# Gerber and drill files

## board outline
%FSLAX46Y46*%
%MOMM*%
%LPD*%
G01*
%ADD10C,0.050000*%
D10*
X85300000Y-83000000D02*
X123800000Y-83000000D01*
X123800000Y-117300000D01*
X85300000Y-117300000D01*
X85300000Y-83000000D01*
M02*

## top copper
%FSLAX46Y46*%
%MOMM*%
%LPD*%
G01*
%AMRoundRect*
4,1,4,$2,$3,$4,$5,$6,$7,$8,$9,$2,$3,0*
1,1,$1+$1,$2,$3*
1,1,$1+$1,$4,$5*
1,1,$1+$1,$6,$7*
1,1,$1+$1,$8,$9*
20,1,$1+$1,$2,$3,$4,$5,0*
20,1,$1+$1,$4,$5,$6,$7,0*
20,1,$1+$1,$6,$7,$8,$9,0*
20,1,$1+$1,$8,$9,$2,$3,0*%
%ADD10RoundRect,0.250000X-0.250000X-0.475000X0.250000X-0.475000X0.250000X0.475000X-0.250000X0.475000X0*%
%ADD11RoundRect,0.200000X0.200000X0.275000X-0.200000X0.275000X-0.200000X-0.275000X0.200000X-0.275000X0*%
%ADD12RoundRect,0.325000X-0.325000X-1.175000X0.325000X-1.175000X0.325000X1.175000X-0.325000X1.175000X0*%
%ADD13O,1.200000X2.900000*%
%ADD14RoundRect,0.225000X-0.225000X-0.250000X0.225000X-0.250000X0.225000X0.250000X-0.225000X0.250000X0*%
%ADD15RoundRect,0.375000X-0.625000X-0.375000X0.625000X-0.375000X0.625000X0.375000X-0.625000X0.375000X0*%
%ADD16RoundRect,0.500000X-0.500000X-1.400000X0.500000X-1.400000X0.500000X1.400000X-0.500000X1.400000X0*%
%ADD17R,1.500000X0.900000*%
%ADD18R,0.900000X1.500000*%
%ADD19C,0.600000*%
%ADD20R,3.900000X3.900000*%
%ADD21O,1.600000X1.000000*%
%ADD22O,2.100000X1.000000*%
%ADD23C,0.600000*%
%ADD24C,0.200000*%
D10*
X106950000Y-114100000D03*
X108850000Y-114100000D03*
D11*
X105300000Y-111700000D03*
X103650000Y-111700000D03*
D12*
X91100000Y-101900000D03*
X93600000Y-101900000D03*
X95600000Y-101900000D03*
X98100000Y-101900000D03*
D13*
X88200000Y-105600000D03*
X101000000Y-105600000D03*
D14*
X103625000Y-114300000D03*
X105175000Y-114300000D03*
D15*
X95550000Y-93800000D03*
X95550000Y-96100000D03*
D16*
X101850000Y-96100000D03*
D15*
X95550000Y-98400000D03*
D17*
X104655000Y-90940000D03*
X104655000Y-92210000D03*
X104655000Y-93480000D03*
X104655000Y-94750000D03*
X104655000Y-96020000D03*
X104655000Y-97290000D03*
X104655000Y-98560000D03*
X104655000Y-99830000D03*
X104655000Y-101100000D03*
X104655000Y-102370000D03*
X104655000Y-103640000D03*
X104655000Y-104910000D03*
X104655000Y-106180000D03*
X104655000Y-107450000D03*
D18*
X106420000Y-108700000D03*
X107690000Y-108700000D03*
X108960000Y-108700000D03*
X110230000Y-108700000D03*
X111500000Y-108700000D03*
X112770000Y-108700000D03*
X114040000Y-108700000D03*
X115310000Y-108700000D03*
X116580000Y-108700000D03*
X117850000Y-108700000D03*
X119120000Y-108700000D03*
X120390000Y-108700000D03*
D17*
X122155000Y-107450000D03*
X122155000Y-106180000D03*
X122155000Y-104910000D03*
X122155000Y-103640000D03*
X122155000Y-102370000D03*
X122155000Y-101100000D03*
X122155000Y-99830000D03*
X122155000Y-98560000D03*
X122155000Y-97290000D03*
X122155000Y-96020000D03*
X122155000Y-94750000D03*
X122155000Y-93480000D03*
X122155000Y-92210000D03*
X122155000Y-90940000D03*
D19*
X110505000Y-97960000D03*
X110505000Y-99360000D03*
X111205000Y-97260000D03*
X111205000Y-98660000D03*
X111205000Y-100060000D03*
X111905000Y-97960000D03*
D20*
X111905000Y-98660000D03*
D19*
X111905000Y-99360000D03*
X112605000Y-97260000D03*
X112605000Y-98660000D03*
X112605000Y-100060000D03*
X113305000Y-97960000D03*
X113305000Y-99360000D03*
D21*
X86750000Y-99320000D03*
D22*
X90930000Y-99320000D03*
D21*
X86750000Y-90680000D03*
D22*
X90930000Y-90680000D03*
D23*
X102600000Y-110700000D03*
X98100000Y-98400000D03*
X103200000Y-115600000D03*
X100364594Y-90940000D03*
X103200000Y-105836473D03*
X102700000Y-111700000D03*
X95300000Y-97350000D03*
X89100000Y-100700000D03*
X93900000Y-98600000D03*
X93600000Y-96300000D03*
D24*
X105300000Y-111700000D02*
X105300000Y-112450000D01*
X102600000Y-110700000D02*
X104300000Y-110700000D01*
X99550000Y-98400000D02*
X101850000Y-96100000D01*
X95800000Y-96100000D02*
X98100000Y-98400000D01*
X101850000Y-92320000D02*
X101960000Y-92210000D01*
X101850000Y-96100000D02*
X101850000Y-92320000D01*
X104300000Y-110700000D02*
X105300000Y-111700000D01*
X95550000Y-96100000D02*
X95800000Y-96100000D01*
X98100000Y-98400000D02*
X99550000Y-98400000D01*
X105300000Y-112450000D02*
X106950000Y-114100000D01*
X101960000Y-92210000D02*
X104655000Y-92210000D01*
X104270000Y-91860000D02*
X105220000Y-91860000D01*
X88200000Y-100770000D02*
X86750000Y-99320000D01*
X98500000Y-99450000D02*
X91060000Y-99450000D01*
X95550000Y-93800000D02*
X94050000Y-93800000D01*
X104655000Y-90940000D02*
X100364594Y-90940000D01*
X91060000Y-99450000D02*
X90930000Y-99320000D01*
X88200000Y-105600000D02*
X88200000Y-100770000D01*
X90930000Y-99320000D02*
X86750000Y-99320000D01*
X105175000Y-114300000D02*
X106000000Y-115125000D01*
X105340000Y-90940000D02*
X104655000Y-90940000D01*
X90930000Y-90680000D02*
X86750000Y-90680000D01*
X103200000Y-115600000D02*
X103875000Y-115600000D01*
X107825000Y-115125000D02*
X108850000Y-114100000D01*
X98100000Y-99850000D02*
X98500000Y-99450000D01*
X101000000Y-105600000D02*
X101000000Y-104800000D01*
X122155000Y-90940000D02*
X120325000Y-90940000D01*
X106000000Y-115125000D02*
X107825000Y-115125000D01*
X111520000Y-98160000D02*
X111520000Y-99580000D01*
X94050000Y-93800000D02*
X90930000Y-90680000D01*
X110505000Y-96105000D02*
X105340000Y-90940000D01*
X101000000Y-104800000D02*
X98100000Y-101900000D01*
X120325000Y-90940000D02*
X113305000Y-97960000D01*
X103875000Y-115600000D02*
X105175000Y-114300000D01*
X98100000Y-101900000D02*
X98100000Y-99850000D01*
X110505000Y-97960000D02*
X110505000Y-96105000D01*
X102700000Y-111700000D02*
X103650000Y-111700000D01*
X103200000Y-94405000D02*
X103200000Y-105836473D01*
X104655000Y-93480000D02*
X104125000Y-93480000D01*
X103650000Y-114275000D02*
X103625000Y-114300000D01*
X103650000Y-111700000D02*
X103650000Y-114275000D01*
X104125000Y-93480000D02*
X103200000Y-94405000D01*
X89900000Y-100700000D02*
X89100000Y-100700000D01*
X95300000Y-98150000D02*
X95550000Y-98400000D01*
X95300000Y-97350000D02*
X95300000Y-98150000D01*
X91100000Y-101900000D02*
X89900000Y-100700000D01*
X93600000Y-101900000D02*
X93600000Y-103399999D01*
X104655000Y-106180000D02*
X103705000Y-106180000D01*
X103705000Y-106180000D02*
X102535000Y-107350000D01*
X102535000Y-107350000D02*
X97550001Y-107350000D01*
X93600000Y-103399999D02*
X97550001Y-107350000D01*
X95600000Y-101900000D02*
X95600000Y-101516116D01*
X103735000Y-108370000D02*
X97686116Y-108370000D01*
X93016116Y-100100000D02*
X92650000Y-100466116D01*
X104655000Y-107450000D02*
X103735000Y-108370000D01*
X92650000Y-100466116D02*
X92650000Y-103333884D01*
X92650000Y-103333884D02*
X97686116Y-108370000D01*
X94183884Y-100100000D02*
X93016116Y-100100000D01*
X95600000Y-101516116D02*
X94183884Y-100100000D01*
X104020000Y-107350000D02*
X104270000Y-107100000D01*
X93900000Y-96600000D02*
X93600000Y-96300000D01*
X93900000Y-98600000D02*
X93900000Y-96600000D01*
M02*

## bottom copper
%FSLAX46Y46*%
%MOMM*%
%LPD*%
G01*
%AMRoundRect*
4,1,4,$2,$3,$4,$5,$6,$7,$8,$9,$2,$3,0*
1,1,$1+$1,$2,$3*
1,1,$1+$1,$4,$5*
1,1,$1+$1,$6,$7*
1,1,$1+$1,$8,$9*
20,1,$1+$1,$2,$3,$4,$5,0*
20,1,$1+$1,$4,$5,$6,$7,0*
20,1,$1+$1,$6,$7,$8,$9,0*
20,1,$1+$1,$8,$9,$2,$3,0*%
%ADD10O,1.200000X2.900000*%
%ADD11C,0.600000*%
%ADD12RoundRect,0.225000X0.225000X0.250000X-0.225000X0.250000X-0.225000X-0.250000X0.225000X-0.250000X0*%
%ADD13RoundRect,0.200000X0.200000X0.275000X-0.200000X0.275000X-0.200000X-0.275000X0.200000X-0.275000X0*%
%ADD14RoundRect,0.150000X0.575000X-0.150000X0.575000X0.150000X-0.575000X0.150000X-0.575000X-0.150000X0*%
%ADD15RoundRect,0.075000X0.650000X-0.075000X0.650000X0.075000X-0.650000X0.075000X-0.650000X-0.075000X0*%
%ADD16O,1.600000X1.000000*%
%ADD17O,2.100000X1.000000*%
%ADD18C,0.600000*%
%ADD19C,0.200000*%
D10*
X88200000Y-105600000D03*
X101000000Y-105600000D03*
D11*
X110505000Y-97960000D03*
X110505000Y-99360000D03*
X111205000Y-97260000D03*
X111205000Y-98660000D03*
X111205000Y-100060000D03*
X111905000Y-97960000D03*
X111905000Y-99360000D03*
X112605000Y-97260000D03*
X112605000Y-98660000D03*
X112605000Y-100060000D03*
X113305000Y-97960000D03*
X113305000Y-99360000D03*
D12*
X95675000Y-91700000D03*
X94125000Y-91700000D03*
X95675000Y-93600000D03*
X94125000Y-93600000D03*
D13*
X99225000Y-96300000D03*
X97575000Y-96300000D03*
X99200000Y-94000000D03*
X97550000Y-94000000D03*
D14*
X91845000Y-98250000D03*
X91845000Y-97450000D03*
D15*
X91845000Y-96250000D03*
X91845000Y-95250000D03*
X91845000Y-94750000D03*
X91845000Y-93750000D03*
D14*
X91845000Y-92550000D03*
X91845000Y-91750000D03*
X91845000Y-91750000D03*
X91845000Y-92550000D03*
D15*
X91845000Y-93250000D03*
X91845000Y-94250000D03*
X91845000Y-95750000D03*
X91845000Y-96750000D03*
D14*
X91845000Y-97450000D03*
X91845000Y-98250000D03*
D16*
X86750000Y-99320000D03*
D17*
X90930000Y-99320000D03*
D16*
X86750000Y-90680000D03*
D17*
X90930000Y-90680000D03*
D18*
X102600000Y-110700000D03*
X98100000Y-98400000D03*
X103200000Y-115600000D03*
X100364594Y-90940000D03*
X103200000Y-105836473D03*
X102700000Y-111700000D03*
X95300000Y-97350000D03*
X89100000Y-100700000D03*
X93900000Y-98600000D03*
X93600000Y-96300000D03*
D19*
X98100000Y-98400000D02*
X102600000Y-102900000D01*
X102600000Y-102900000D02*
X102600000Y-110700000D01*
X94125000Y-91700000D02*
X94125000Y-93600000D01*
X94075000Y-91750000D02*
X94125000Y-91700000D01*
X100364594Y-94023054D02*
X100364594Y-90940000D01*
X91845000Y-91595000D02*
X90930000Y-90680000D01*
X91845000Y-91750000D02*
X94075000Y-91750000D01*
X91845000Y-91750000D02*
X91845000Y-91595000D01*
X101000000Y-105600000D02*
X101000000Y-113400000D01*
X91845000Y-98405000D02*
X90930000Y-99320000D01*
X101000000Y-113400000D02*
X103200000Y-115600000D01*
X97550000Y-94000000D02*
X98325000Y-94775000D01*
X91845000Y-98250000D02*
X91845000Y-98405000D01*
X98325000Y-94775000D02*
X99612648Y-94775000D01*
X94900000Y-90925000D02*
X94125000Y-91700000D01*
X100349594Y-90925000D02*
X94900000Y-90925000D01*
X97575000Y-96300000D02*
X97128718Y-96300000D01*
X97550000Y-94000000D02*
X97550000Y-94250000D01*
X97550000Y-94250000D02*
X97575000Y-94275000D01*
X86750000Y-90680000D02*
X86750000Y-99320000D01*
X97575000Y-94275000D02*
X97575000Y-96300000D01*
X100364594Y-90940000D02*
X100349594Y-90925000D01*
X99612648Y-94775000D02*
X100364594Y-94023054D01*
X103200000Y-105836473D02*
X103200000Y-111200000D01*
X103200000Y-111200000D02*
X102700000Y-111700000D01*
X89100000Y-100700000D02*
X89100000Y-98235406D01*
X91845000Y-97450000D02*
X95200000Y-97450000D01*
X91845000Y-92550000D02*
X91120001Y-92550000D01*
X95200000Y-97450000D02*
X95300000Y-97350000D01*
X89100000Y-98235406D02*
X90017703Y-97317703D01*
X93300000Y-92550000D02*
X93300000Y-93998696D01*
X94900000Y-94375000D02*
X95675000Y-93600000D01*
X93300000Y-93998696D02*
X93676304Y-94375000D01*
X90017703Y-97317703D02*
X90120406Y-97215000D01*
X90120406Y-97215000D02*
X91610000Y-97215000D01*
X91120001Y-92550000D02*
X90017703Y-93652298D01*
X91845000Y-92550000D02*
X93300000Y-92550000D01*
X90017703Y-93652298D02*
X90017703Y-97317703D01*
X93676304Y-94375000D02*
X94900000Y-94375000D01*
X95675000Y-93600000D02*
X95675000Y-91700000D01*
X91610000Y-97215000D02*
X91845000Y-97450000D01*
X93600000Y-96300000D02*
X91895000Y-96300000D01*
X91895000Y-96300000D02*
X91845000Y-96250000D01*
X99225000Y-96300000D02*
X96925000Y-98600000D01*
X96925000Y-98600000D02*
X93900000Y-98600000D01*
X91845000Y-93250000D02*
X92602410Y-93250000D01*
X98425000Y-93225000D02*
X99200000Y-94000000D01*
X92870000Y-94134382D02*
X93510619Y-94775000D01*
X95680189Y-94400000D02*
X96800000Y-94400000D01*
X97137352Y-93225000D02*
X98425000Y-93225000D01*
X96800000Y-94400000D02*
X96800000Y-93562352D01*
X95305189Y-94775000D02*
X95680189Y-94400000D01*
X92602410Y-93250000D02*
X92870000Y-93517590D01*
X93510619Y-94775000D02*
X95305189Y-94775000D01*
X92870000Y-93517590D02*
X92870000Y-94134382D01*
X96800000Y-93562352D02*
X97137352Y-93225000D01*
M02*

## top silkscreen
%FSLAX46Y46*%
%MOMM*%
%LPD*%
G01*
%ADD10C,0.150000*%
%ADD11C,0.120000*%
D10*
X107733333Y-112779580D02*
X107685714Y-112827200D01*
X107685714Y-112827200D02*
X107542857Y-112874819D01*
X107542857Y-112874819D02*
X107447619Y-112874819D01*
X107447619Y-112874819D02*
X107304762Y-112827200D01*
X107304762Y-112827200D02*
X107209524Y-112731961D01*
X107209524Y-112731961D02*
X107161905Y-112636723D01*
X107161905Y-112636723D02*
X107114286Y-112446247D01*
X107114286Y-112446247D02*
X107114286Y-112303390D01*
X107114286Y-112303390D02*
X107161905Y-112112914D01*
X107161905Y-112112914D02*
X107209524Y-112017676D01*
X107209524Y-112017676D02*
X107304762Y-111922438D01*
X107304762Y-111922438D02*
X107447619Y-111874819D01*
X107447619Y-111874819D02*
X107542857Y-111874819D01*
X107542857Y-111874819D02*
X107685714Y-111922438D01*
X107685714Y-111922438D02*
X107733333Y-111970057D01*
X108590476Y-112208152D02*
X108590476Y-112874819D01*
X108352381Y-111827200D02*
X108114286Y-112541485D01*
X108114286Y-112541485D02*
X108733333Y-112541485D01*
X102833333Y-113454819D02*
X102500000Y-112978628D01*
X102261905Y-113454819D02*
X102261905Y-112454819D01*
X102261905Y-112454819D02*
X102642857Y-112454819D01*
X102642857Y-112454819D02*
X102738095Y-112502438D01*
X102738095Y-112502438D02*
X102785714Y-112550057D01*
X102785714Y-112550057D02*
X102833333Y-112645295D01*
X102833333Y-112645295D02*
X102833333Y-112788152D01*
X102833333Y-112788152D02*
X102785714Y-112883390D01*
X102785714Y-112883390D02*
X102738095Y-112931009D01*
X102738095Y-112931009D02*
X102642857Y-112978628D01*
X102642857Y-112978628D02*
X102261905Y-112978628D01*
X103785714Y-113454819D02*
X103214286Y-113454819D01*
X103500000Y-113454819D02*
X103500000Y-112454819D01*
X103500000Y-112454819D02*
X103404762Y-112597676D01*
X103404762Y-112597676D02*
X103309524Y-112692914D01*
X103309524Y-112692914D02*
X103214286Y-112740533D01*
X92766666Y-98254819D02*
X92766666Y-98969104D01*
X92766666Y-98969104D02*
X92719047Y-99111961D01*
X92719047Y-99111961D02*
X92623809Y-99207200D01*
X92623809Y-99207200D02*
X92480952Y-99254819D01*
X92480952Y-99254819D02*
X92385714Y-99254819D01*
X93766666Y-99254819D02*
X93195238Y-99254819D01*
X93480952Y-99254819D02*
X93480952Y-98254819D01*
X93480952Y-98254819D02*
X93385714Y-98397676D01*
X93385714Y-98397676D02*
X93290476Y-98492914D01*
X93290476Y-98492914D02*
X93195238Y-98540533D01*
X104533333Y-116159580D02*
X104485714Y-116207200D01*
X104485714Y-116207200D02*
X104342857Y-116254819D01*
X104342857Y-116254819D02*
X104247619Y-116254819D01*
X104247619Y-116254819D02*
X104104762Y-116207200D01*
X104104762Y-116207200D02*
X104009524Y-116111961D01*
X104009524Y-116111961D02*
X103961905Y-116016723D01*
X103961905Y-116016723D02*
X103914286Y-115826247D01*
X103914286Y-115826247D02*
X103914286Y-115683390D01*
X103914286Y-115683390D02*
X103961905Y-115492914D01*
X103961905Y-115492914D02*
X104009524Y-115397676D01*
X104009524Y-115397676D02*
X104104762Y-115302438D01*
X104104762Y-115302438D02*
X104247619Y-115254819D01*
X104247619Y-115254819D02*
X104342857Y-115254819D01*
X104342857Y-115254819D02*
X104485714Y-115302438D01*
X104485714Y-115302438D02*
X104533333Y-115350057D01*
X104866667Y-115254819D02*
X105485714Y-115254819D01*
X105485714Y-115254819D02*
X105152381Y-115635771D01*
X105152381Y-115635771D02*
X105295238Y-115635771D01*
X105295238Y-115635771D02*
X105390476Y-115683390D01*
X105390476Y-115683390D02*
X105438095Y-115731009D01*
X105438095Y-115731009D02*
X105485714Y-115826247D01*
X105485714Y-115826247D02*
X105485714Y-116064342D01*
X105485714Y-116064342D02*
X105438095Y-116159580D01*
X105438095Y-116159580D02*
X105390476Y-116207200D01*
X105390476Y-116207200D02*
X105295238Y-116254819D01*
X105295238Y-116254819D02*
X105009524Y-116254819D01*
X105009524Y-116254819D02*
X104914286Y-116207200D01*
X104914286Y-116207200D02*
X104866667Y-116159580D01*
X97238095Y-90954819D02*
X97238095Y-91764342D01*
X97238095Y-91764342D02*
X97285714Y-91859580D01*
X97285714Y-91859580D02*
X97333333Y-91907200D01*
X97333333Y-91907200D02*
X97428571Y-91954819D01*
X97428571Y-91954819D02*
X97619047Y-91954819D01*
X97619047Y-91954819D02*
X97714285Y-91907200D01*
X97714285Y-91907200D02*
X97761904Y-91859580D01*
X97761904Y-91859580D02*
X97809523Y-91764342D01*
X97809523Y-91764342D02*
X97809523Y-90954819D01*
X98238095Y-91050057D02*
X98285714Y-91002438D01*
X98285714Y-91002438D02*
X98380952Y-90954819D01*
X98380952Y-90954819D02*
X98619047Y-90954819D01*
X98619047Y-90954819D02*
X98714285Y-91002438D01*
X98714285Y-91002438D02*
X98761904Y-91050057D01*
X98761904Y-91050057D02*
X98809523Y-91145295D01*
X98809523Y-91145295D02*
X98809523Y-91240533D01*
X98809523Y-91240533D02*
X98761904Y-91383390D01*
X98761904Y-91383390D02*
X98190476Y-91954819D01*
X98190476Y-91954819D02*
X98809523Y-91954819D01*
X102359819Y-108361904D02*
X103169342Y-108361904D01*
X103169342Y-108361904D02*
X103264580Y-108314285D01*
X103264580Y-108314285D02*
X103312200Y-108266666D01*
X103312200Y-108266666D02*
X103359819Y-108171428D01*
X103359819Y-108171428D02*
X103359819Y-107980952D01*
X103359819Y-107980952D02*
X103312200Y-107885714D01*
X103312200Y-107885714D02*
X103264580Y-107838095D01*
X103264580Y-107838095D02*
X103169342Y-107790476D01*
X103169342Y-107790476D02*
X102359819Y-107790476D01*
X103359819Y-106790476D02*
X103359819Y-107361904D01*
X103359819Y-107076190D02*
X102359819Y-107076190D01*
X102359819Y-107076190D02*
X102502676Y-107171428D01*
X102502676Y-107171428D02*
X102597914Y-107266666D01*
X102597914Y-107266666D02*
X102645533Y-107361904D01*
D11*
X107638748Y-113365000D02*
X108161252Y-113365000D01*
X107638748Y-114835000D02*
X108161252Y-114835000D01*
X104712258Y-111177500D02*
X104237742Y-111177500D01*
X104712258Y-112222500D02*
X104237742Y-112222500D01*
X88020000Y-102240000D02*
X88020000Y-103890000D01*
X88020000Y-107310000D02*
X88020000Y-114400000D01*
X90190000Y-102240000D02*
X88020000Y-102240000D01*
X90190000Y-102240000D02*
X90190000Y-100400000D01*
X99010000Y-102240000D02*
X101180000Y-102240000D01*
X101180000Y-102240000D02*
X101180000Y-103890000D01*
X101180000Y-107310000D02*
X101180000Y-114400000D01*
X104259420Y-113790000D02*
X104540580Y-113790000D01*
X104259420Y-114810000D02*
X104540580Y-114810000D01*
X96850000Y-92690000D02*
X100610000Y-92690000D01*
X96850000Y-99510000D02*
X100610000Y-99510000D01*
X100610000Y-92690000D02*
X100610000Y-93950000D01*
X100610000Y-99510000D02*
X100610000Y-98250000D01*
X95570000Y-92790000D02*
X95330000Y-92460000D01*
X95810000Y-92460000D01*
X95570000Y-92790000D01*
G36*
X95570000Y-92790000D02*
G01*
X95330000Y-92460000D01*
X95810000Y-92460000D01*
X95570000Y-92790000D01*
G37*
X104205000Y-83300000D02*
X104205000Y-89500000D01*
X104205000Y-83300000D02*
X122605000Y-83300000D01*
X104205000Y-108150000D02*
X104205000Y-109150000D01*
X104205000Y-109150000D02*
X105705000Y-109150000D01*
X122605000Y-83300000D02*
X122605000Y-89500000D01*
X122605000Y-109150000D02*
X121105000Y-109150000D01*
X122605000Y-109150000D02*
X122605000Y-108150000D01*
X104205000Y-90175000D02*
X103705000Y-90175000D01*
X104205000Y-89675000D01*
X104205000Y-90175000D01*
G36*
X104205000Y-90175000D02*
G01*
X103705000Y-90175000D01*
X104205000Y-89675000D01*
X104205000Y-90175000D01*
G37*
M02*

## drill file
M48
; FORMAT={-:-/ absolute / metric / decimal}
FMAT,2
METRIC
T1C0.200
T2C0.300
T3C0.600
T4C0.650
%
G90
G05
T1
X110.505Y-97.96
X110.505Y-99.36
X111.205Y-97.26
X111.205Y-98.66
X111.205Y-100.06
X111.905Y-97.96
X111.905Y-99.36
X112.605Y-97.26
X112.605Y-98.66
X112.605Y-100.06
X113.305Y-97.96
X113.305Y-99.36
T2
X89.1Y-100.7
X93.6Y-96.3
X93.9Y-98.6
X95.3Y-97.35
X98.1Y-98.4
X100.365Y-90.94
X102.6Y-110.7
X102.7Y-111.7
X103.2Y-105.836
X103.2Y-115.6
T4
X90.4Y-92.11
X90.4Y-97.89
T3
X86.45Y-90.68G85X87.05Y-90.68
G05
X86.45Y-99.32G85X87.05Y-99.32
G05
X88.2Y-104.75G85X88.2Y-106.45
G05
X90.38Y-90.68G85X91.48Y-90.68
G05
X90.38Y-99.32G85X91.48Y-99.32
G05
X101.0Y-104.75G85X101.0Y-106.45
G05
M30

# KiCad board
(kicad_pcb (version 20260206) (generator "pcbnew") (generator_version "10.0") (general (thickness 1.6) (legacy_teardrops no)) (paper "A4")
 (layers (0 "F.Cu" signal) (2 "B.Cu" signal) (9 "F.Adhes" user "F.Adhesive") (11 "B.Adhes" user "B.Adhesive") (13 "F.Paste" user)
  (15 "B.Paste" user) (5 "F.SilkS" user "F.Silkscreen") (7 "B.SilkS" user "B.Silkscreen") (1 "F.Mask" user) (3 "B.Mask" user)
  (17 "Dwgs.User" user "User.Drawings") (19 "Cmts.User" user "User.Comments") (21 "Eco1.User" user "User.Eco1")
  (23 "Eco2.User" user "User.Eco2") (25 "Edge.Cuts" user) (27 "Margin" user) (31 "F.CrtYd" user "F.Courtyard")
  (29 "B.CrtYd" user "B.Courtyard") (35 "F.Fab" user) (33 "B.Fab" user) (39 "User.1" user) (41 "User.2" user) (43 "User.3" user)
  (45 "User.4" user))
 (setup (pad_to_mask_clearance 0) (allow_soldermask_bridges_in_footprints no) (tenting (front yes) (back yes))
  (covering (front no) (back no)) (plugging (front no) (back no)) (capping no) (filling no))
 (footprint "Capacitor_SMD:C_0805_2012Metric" (layer "F.Cu") (at 107.9 114.1)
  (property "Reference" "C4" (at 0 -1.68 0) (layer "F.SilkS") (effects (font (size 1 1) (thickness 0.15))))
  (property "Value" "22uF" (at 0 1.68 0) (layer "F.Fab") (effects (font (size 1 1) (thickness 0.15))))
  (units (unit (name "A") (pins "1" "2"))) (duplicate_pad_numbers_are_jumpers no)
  (fp_line (start -0.261252 -0.735) (end 0.261252 -0.735) (stroke (width 0.12) (type solid)) (layer "F.SilkS"))
  (fp_line (start -0.261252 0.735) (end 0.261252 0.735) (stroke (width 0.12) (type solid)) (layer "F.SilkS"))
  (pad "1" smd roundrect (at -0.95 0) (size 1 1.45) (layers "F.Cu" "F.Mask" "F.Paste") (roundrect_rratio 0.25) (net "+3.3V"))
  (pad "2" smd roundrect (at 0.95 0) (size 1 1.45) (layers "F.Cu" "F.Mask" "F.Paste") (roundrect_rratio 0.25) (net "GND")))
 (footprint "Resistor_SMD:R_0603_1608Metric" (layer "F.Cu") (at 104.475 111.7 180)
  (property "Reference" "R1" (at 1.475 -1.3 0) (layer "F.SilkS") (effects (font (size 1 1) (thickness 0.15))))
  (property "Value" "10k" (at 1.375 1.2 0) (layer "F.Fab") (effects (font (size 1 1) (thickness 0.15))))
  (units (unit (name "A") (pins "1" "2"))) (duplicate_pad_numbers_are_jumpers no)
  (fp_line (start -0.237258 0.5225) (end 0.237258 0.5225) (stroke (width 0.12) (type solid)) (layer "F.SilkS"))
  (fp_line (start -0.237258 -0.5225) (end 0.237258 -0.5225) (stroke (width 0.12) (type solid)) (layer "F.SilkS"))
  (pad "1" smd roundrect (at -0.825 0 180) (size 0.8 0.95) (layers "F.Cu" "F.Mask" "F.Paste") (roundrect_rratio 0.25) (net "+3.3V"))
  (pad "2" smd roundrect (at 0.825 0 180) (size 0.8 0.95) (layers "F.Cu" "F.Mask" "F.Paste") (roundrect_rratio 0.25) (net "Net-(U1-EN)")))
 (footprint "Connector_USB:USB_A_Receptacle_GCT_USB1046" (layer "F.Cu") (at 94.6 109.15)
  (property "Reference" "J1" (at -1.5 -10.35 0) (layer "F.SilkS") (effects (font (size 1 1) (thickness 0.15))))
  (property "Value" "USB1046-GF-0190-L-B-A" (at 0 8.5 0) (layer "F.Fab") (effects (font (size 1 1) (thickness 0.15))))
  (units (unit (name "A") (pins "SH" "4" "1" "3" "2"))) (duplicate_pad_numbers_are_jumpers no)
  (fp_line (start -6.58 -6.91) (end -6.58 -5.26) (stroke (width 0.12) (type default)) (layer "F.SilkS"))
  (fp_line (start -6.58 -1.84) (end -6.58 5.25) (stroke (width 0.12) (type default)) (layer "F.SilkS"))
  (fp_line (start -4.41 -6.91) (end -6.58 -6.91) (stroke (width 0.12) (type default)) (layer "F.SilkS"))
  (fp_line (start -4.41 -6.91) (end -4.41 -8.75) (stroke (width 0.12) (type default)) (layer "F.SilkS"))
  (fp_line (start 4.41 -6.91) (end 6.58 -6.91) (stroke (width 0.12) (type default)) (layer "F.SilkS"))
  (fp_line (start 6.58 -6.91) (end 6.58 -5.26) (stroke (width 0.12) (type default)) (layer "F.SilkS"))
  (fp_line (start 6.58 -1.84) (end 6.58 5.25) (stroke (width 0.12) (type default)) (layer "F.SilkS"))
  (pad "" smd oval (at -6.4 -3.55) (size 1.2 2.9) (layers "F.Paste") (thermal_bridge_angle 45))
  (pad "" smd oval (at 6.4 -3.55) (size 1.2 2.9) (layers "F.Paste") (thermal_bridge_angle 45))
  (pad "1" smd roundrect (at -3.5 -7.25) (size 1.3 3) (layers "F.Cu" "F.Mask" "F.Paste") (roundrect_rratio 0.25) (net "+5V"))
  (pad "2" smd roundrect (at -1 -7.25) (size 1.3 3) (layers "F.Cu" "F.Mask" "F.Paste") (roundrect_rratio 0.25) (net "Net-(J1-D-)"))
  (pad "3" smd roundrect (at 1 -7.25) (size 1.3 3) (layers "F.Cu" "F.Mask" "F.Paste") (roundrect_rratio 0.25) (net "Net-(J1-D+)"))
  (pad "4" smd roundrect (at 3.5 -7.25) (size 1.3 3) (layers "F.Cu" "F.Mask" "F.Paste") (roundrect_rratio 0.25) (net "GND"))
  (pad "SH" thru_hole oval (at -6.4 -3.55) (size 1.2 2.9) (drill oval 0.6 2.3) (layers "*.Cu" "*.Mask") (remove_unused_layers no)
   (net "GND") (thermal_bridge_angle 45))
  (pad "SH" thru_hole oval (at 6.4 -3.55) (size 1.2 2.9) (drill oval 0.6 2.3) (layers "*.Cu" "*.Mask") (remove_unused_layers no) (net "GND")
   (thermal_bridge_angle 45)))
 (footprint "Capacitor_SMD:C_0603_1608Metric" (layer "F.Cu") (at 104.4 114.3)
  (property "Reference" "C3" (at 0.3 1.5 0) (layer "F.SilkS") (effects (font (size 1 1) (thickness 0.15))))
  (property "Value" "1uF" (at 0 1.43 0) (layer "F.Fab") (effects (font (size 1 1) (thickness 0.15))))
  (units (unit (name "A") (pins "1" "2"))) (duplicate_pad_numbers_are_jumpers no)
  (fp_line (start -0.14058 -0.51) (end 0.14058 -0.51) (stroke (width 0.12) (type solid)) (layer "F.SilkS"))
  (fp_line (start -0.14058 0.51) (end 0.14058 0.51) (stroke (width 0.12) (type solid)) (layer "F.SilkS"))
  (pad "1" smd roundrect (at -0.775 0) (size 0.9 0.95) (layers "F.Cu" "F.Mask" "F.Paste") (roundrect_rratio 0.25) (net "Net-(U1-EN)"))
  (pad "2" smd roundrect (at 0.775 0) (size 0.9 0.95) (layers "F.Cu" "F.Mask" "F.Paste") (roundrect_rratio 0.25) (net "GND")))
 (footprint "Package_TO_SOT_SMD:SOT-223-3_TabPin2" (layer "F.Cu") (at 98.7 96.1)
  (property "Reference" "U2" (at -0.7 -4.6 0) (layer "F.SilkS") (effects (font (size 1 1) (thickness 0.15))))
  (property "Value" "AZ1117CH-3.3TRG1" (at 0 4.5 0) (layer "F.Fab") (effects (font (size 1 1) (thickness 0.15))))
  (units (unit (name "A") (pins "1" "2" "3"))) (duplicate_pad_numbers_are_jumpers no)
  (fp_line (start -1.85 -3.41) (end 1.91 -3.41) (stroke (width 0.12) (type solid)) (layer "F.SilkS"))
  (fp_line (start -1.85 3.41) (end 1.91 3.41) (stroke (width 0.12) (type solid)) (layer "F.SilkS"))
  (fp_line (start 1.91 -3.41) (end 1.91 -2.15) (stroke (width 0.12) (type solid)) (layer "F.SilkS"))
  (fp_line (start 1.91 3.41) (end 1.91 2.15) (stroke (width 0.12) (type solid)) (layer "F.SilkS"))
  (fp_poly
   (pts (xy -3.13 -3.31) (xy -3.37 -3.64) (xy -2.89 -3.64) (xy -3.13 -3.31)) (stroke (width 0.12) (type solid)) (fill yes) (layer "F.SilkS"))
  (pad "1" smd roundrect (at -3.15 -2.3) (size 2 1.5) (layers "F.Cu" "F.Mask" "F.Paste") (roundrect_rratio 0.25) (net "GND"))
  (pad "2" smd roundrect (at -3.15 0) (size 2 1.5) (layers "F.Cu" "F.Mask" "F.Paste") (roundrect_rratio 0.25) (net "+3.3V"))
  (pad "2" smd roundrect (at 3.15 0) (size 2 3.8) (layers "F.Cu" "F.Mask" "F.Paste") (roundrect_rratio 0.25) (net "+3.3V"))
  (pad "3" smd roundrect (at -3.15 2.3) (size 2 1.5) (layers "F.Cu" "F.Mask" "F.Paste") (roundrect_rratio 0.25) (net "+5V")))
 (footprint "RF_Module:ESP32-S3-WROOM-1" (layer "F.Cu") (at 113.405 96.2)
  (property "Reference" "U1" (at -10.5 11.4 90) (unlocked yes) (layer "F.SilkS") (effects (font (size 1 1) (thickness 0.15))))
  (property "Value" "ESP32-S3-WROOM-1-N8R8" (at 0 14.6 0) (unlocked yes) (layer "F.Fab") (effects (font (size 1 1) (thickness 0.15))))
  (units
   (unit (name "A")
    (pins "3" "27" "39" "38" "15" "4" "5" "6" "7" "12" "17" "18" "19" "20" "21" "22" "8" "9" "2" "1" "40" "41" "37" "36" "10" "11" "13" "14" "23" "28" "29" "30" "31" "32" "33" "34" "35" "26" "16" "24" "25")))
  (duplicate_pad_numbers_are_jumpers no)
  (fp_line (start -9.2 -12.9) (end -9.2 -6.7) (stroke (width 0.12) (type solid)) (layer "F.SilkS"))
  (fp_line (start -9.2 -12.9) (end 9.2 -12.9) (stroke (width 0.12) (type solid)) (layer "F.SilkS"))
  (fp_line (start -9.2 11.95) (end -9.2 12.95) (stroke (width 0.12) (type solid)) (layer "F.SilkS"))
  (fp_line (start -9.2 12.95) (end -7.7 12.95) (stroke (width 0.12) (type solid)) (layer "F.SilkS"))
  (fp_line (start 9.2 -12.9) (end 9.2 -6.7) (stroke (width 0.12) (type solid)) (layer "F.SilkS"))
  (fp_line (start 9.2 12.95) (end 7.7 12.95) (stroke (width 0.12) (type solid)) (layer "F.SilkS"))
  (fp_line (start 9.2 12.95) (end 9.2 11.95) (stroke (width 0.12) (type solid)) (layer "F.SilkS"))
  (fp_poly
   (pts (xy -9.2 -6.025) (xy -9.7 -6.025) (xy -9.2 -6.525) (xy -9.2 -6.025)) (stroke (width 0.12) (type solid)) (fill yes) (layer "F.SilkS"))
  (pad "" smd rect (at -2.9 1.06) (size 0.9 0.9) (layers "F.Paste"))
  (pad "" smd rect (at -2.9 2.46 270) (size 0.9 0.9) (layers "F.Paste"))
  (pad "" smd rect (at -2.9 3.86) (size 0.9 0.9) (layers "F.Paste"))
  (pad "" smd rect (at -1.5 1.06 270) (size 0.9 0.9) (layers "F.Paste"))
  (pad "" smd rect (at -1.5 2.46 270) (size 0.9 0.9) (layers "F.Paste"))
  (pad "" smd rect (at -1.5 3.86 270) (size 0.9 0.9) (layers "F.Paste"))
  (pad "" smd rect (at -0.1 1.06 270) (size 0.9 0.9) (layers "F.Paste"))
  (pad "" smd rect (at -0.1 2.46 270) (size 0.9 0.9) (layers "F.Paste"))
  (pad "" smd rect (at -0.1 3.86 270) (size 0.9 0.9) (layers "F.Paste"))
  (pad "1" smd rect (at -8.75 -5.26) (size 1.5 0.9) (layers "F.Cu" "F.Mask" "F.Paste") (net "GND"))
  (pad "2" smd rect (at -8.75 -3.99) (size 1.5 0.9) (layers "F.Cu" "F.Mask" "F.Paste") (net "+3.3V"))
  (pad "3" smd rect (at -8.75 -2.72) (size 1.5 0.9) (layers "F.Cu" "F.Mask" "F.Paste") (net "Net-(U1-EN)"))
  (pad "4" smd rect (at -8.75 -1.45) (size 1.5 0.9) (layers "F.Cu" "F.Mask" "F.Paste") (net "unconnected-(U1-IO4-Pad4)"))
  (pad "5" smd rect (at -8.75 -0.18) (size 1.5 0.9) (layers "F.Cu" "F.Mask" "F.Paste") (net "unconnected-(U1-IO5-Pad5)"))
  (pad "6" smd rect (at -8.75 1.09) (size 1.5 0.9) (layers "F.Cu" "F.Mask" "F.Paste") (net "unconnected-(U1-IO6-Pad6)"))
  (pad "7" smd rect (at -8.75 2.36) (size 1.5 0.9) (layers "F.Cu" "F.Mask" "F.Paste") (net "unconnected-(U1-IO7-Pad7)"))
  (pad "8" smd rect (at -8.75 3.63) (size 1.5 0.9) (layers "F.Cu" "F.Mask" "F.Paste") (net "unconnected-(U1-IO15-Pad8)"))
  (pad "9" smd rect (at -8.75 4.9) (size 1.5 0.9) (layers "F.Cu" "F.Mask" "F.Paste") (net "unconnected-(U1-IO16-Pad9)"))
  (pad "10" smd rect (at -8.75 6.17) (size 1.5 0.9) (layers "F.Cu" "F.Mask" "F.Paste") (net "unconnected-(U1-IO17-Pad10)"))
  (pad "11" smd rect (at -8.75 7.44) (size 1.5 0.9) (layers "F.Cu" "F.Mask" "F.Paste") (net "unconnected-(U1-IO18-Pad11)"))
  (pad "12" smd rect (at -8.75 8.71) (size 1.5 0.9) (layers "F.Cu" "F.Mask" "F.Paste") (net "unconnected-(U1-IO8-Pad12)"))
  (pad "13" smd rect (at -8.75 9.98) (size 1.5 0.9) (layers "F.Cu" "F.Mask" "F.Paste") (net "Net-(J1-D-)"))
  (pad "14" smd rect (at -8.75 11.25 180) (size 1.5 0.9) (layers "F.Cu" "F.Mask" "F.Paste") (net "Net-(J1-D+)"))
  (pad "15" smd rect (at -6.985 12.5 270) (size 1.5 0.9) (layers "F.Cu" "F.Mask" "F.Paste") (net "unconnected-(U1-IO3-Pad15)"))
  (pad "16" smd rect (at -5.715 12.5 270) (size 1.5 0.9) (layers "F.Cu" "F.Mask" "F.Paste") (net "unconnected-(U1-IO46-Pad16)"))
  (pad "17" smd rect (at -4.445 12.5 270) (size 1.5 0.9) (layers "F.Cu" "F.Mask" "F.Paste") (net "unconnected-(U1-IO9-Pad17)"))
  (pad "18" smd rect (at -3.175 12.5 270) (size 1.5 0.9) (layers "F.Cu" "F.Mask" "F.Paste") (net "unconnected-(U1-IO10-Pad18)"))
  (pad "19" smd rect (at -1.905 12.5 270) (size 1.5 0.9) (layers "F.Cu" "F.Mask" "F.Paste") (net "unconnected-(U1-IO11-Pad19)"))
  (pad "20" smd rect (at -0.635 12.5 270) (size 1.5 0.9) (layers "F.Cu" "F.Mask" "F.Paste") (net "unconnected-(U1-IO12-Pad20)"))
  (pad "21" smd rect (at 0.635 12.5 270) (size 1.5 0.9) (layers "F.Cu" "F.Mask" "F.Paste") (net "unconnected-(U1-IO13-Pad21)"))
  (pad "22" smd rect (at 1.905 12.5 270) (size 1.5 0.9) (layers "F.Cu" "F.Mask" "F.Paste") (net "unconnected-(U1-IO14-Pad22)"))
  (pad "23" smd rect (at 3.175 12.5 270) (size 1.5 0.9) (layers "F.Cu" "F.Mask" "F.Paste") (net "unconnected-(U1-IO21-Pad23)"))
  (pad "24" smd rect (at 4.445 12.5 270) (size 1.5 0.9) (layers "F.Cu" "F.Mask" "F.Paste") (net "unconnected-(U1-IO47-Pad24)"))
  (pad "25" smd rect (at 5.715 12.5 270) (size 1.5 0.9) (layers "F.Cu" "F.Mask" "F.Paste") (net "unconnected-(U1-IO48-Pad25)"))
  (pad "26" smd rect (at 6.985 12.5 270) (size 1.5 0.9) (layers "F.Cu" "F.Mask" "F.Paste") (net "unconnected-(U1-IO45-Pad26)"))
  (pad "27" smd rect (at 8.75 11.25) (size 1.5 0.9) (layers "F.Cu" "F.Mask" "F.Paste") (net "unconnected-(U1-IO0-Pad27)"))
  (pad "28" smd rect (at 8.75 9.98) (size 1.5 0.9) (layers "F.Cu" "F.Mask" "F.Paste") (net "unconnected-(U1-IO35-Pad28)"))
  (pad "29" smd rect (at 8.75 8.71) (size 1.5 0.9) (layers "F.Cu" "F.Mask" "F.Paste") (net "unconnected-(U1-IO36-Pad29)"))
  (pad "30" smd rect (at 8.75 7.44) (size 1.5 0.9) (layers "F.Cu" "F.Mask" "F.Paste") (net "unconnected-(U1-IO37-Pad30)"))
  (pad "31" smd rect (at 8.75 6.17) (size 1.5 0.9) (layers "F.Cu" "F.Mask" "F.Paste") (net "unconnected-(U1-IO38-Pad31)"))
  (pad "32" smd rect (at 8.75 4.9) (size 1.5 0.9) (layers "F.Cu" "F.Mask" "F.Paste") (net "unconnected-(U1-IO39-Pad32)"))
  (pad "33" smd rect (at 8.75 3.63) (size 1.5 0.9) (layers "F.Cu" "F.Mask" "F.Paste") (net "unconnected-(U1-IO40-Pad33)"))
  (pad "34" smd rect (at 8.75 2.36) (size 1.5 0.9) (layers "F.Cu" "F.Mask" "F.Paste") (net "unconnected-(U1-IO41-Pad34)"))
  (pad "35" smd rect (at 8.75 1.09) (size 1.5 0.9) (layers "F.Cu" "F.Mask" "F.Paste") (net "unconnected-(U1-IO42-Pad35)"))
  (pad "36" smd rect (at 8.75 -0.18) (size 1.5 0.9) (layers "F.Cu" "F.Mask" "F.Paste") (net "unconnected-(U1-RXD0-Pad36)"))
  (pad "37" smd rect (at 8.75 -1.45) (size 1.5 0.9) (layers "F.Cu" "F.Mask" "F.Paste") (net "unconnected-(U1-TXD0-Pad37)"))
  (pad "38" smd rect (at 8.75 -2.72) (size 1.5 0.9) (layers "F.Cu" "F.Mask" "F.Paste") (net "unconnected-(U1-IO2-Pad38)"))
  (pad "39" smd rect (at 8.75 -3.99) (size 1.5 0.9) (layers "F.Cu" "F.Mask" "F.Paste") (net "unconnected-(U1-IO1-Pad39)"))
  (pad "40" smd rect (at 8.75 -5.26) (size 1.5 0.9) (layers "F.Cu" "F.Mask" "F.Paste") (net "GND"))
  (pad "41" thru_hole circle (at -2.9 1.76 90) (size 0.6 0.6) (drill 0.2) (layers "*.Cu" "F.Mask") (remove_unused_layers no) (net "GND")
   (zone_connect 2))
  (pad "41" thru_hole circle (at -2.9 3.16) (size 0.6 0.6) (drill 0.2) (layers "*.Cu" "F.Mask") (remove_unused_layers no) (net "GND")
   (zone_connect 2))
  (pad "41" thru_hole circle (at -2.2 1.06) (size 0.6 0.6) (drill 0.2) (layers "*.Cu" "F.Mask") (remove_unused_layers no) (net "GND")
   (zone_connect 2))
  (pad "41" thru_hole circle (at -2.2 2.46) (size 0.6 0.6) (drill 0.2) (layers "*.Cu" "F.Mask") (remove_unused_layers no) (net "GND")
   (zone_connect 2))
  (pad "41" thru_hole circle (at -2.2 3.86) (size 0.6 0.6) (drill 0.2) (layers "*.Cu" "F.Mask") (remove_unused_layers no) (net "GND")
   (zone_connect 2))
  (pad "41" thru_hole circle (at -1.5 1.76) (size 0.6 0.6) (drill 0.2) (layers "*.Cu" "F.Mask") (remove_unused_layers no) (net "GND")
   (zone_connect 2))
  (pad "41" smd rect (at -1.5 2.46 270) (size 3.9 3.9) (layers "F.Cu" "F.Mask") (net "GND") (zone_connect 2))
  (pad "41" thru_hole circle (at -1.5 3.16) (size 0.6 0.6) (drill 0.2) (layers "*.Cu" "F.Mask") (remove_unused_layers no) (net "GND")
   (zone_connect 2))
  (pad "41" thru_hole circle (at -0.8 1.06) (size 0.6 0.6) (drill 0.2) (layers "*.Cu" "F.Mask") (remove_unused_layers no) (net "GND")
   (zone_connect 2))
  (pad "41" thru_hole circle (at -0.8 2.46) (size 0.6 0.6) (drill 0.2) (layers "*.Cu" "F.Mask") (remove_unused_layers no) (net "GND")
   (zone_connect 2))
  (pad "41" thru_hole circle (at -0.8 3.86) (size 0.6 0.6) (drill 0.2) (layers "*.Cu" "F.Mask") (remove_unused_layers no) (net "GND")
   (zone_connect 2))
  (pad "41" thru_hole circle (at -0.1 1.76) (size 0.6 0.6) (drill 0.2) (layers "*.Cu" "F.Mask") (remove_unused_layers no) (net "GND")
   (zone_connect 2))
  (pad "41" thru_hole circle (at -0.1 3.16) (size 0.6 0.6) (drill 0.2) (layers "*.Cu" "F.Mask") (remove_unused_layers no) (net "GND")
   (zone_connect 2))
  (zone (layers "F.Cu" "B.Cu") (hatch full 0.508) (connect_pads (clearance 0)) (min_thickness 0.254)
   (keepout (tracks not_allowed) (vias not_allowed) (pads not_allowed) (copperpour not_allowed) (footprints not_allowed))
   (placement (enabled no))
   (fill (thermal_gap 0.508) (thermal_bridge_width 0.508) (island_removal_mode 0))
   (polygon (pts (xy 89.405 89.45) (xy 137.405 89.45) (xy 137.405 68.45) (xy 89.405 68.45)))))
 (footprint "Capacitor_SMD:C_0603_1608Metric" (layer "B.Cu") (at 94.9 91.7 180)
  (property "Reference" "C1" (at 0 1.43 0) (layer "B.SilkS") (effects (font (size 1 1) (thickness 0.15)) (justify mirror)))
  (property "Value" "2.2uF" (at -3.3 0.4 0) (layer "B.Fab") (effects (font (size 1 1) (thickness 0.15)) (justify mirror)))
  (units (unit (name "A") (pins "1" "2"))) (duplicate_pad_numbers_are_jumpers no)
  (pad "1" smd roundrect (at -0.775 0 180) (size 0.9 0.95) (layers "B.Cu" "B.Mask" "B.Paste") (roundrect_rratio 0.25) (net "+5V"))
  (pad "2" smd roundrect (at 0.775 0 180) (size 0.9 0.95) (layers "B.Cu" "B.Mask" "B.Paste") (roundrect_rratio 0.25) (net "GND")))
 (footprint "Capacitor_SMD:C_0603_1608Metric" (layer "B.Cu") (at 94.9 93.6 180)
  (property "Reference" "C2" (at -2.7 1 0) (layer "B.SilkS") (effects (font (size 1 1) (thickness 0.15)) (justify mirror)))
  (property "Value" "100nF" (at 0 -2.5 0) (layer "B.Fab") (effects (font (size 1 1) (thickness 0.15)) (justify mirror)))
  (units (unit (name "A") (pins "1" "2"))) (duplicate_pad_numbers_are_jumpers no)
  (pad "1" smd roundrect (at -0.775 0 180) (size 0.9 0.95) (layers "B.Cu" "B.Mask" "B.Paste") (roundrect_rratio 0.25) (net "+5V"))
  (pad "2" smd roundrect (at 0.775 0 180) (size 0.9 0.95) (layers "B.Cu" "B.Mask" "B.Paste") (roundrect_rratio 0.25) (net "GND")))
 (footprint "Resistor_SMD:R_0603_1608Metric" (layer "B.Cu") (at 98.4 96.3 180)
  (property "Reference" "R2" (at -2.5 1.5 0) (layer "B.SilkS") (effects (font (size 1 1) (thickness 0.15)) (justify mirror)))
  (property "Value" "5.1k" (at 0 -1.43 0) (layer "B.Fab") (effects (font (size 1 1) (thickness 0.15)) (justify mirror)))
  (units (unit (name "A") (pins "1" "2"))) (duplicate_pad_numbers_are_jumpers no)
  (pad "1" smd roundrect (at -0.825 0 180) (size 0.8 0.95) (layers "B.Cu" "B.Mask" "B.Paste") (roundrect_rratio 0.25) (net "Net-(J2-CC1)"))
  (pad "2" smd roundrect (at 0.825 0 180) (size 0.8 0.95) (layers "B.Cu" "B.Mask" "B.Paste") (roundrect_rratio 0.25) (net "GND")))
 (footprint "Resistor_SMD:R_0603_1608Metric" (layer "B.Cu") (at 98.375 94 180)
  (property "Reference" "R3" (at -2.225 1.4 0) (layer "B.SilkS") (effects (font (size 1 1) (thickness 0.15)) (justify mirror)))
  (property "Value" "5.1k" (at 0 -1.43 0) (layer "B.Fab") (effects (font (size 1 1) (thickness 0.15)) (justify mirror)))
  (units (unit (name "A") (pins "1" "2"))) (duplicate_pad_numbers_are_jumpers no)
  (pad "1" smd roundrect (at -0.825 0 180) (size 0.8 0.95) (layers "B.Cu" "B.Mask" "B.Paste") (roundrect_rratio 0.25) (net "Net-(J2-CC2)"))
  (pad "2" smd roundrect (at 0.825 0 180) (size 0.8 0.95) (layers "B.Cu" "B.Mask" "B.Paste") (roundrect_rratio 0.25) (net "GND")))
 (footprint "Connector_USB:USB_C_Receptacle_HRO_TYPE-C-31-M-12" (layer "B.Cu") (at 87.8 95 90)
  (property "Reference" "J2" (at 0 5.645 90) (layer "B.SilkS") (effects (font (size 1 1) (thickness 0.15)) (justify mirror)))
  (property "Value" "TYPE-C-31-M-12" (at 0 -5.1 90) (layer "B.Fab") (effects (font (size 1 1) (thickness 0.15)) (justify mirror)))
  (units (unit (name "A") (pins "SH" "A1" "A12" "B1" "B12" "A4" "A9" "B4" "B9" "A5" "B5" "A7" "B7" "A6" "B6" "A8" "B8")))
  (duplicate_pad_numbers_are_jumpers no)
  (pad "" np_thru_hole circle (at -2.89 2.6 90) (size 0.65 0.65) (drill 0.65) (layers "*.Cu" "*.Mask"))
  (pad "" np_thru_hole circle (at 2.89 2.6 90) (size 0.65 0.65) (drill 0.65) (layers "*.Cu" "*.Mask"))
  (pad "A1" smd roundrect (at -3.25 4.045 90) (size 0.6 1.45) (layers "B.Cu" "B.Mask" "B.Paste") (roundrect_rratio 0.25) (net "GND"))
  (pad "A4" smd roundrect (at -2.45 4.045 90) (size 0.6 1.45) (layers "B.Cu" "B.Mask" "B.Paste") (roundrect_rratio 0.25) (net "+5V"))
  (pad "A5" smd roundrect (at -1.25 4.045 90) (size 0.3 1.45) (layers "B.Cu" "B.Mask" "B.Paste") (roundrect_rratio 0.25)
   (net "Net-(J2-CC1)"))
  (pad "A6" smd roundrect (at -0.25 4.045 90) (size 0.3 1.45) (layers "B.Cu" "B.Mask" "B.Paste") (roundrect_rratio 0.25)
   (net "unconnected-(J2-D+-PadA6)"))
  (pad "A7" smd roundrect (at 0.25 4.045 90) (size 0.3 1.45) (layers "B.Cu" "B.Mask" "B.Paste") (roundrect_rratio 0.25)
   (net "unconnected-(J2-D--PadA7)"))
  (pad "A8" smd roundrect (at 1.25 4.045 90) (size 0.3 1.45) (layers "B.Cu" "B.Mask" "B.Paste") (roundrect_rratio 0.25)
   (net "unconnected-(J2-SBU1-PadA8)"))
  (pad "A9" smd roundrect (at 2.45 4.045 90) (size 0.6 1.45) (layers "B.Cu" "B.Mask" "B.Paste") (roundrect_rratio 0.25) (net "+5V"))
  (pad "A12" smd roundrect (at 3.25 4.045 90) (size 0.6 1.45) (layers "B.Cu" "B.Mask" "B.Paste") (roundrect_rratio 0.25) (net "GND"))
  (pad "B1" smd roundrect (at 3.25 4.045 90) (size 0.6 1.45) (layers "B.Cu" "B.Mask" "B.Paste") (roundrect_rratio 0.25) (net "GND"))
  (pad "B4" smd roundrect (at 2.45 4.045 90) (size 0.6 1.45) (layers "B.Cu" "B.Mask" "B.Paste") (roundrect_rratio 0.25) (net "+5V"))
  (pad "B5" smd roundrect (at 1.75 4.045 90) (size 0.3 1.45) (layers "B.Cu" "B.Mask" "B.Paste") (roundrect_rratio 0.25) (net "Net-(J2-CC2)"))
  (pad "B6" smd roundrect (at 0.75 4.045 90) (size 0.3 1.45) (layers "B.Cu" "B.Mask" "B.Paste") (roundrect_rratio 0.25)
   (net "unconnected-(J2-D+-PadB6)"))
  (pad "B7" smd roundrect (at -0.75 4.045 90) (size 0.3 1.45) (layers "B.Cu" "B.Mask" "B.Paste") (roundrect_rratio 0.25)
   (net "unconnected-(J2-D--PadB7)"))
  (pad "B8" smd roundrect (at -1.75 4.045 90) (size 0.3 1.45) (layers "B.Cu" "B.Mask" "B.Paste") (roundrect_rratio 0.25)
   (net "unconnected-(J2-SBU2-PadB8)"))
  (pad "B9" smd roundrect (at -2.45 4.045 90) (size 0.6 1.45) (layers "B.Cu" "B.Mask" "B.Paste") (roundrect_rratio 0.25) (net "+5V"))
  (pad "B12" smd roundrect (at -3.25 4.045 90) (size 0.6 1.45) (layers "B.Cu" "B.Mask" "B.Paste") (roundrect_rratio 0.25) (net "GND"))
  (pad "SH" thru_hole oval (at -4.32 -1.05 90) (size 1 1.6) (drill oval 0.6 1.2) (layers "*.Cu" "*.Mask") (remove_unused_layers no)
   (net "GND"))
  (pad "SH" thru_hole oval (at -4.32 3.13 90) (size 1 2.1) (drill oval 0.6 1.7) (layers "*.Cu" "*.Mask") (remove_unused_layers no)
   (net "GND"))
  (pad "SH" thru_hole oval (at 4.32 -1.05 90) (size 1 1.6) (drill oval 0.6 1.2) (layers "*.Cu" "*.Mask") (remove_unused_layers no)
   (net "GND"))
  (pad "SH" thru_hole oval (at 4.32 3.13 90) (size 1 2.1) (drill oval 0.6 1.7) (layers "*.Cu" "*.Mask") (remove_unused_layers no)
   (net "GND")))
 (gr_rect (start 85.3 83) (end 123.8 117.3) (stroke (width 0.05) (type default)) (fill no) (layer "Edge.Cuts"))
 (segment (start 105.3 111.7) (end 105.3 112.45) (width 0.2) (layer "F.Cu") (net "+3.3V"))
 (segment (start 102.6 110.7) (end 104.3 110.7) (width 0.2) (layer "F.Cu") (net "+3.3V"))
 (segment (start 99.55 98.4) (end 101.85 96.1) (width 0.2) (layer "F.Cu") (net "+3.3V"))
 (segment (start 95.8 96.1) (end 98.1 98.4) (width 0.2) (layer "F.Cu") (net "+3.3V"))
 (segment (start 101.85 92.32) (end 101.96 92.21) (width 0.2) (layer "F.Cu") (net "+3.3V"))
 (segment (start 101.85 96.1) (end 101.85 92.32) (width 0.2) (layer "F.Cu") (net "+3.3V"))
 (segment (start 104.3 110.7) (end 105.3 111.7) (width 0.2) (layer "F.Cu") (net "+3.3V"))
 (segment (start 95.55 96.1) (end 95.8 96.1) (width 0.2) (layer "F.Cu") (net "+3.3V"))
 (segment (start 98.1 98.4) (end 99.55 98.4) (width 0.2) (layer "F.Cu") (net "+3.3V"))
 (segment (start 105.3 112.45) (end 106.95 114.1) (width 0.2) (layer "F.Cu") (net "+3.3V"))
 (segment (start 101.96 92.21) (end 104.655 92.21) (width 0.2) (layer "F.Cu") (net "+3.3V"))
 (segment (start 104.27 91.86) (end 105.22 91.86) (width 0.2) (layer "F.Cu") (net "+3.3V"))
 (via (at 102.6 110.7) (size 0.6) (drill 0.3) (layers "F.Cu" "B.Cu") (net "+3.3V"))
 (via (at 98.1 98.4) (size 0.6) (drill 0.3) (layers "F.Cu" "B.Cu") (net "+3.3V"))
 (segment (start 98.1 98.4) (end 102.6 102.9) (width 0.2) (layer "B.Cu") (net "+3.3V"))
 (segment (start 102.6 102.9) (end 102.6 110.7) (width 0.2) (layer "B.Cu") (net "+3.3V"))
 (segment (start 88.2 100.77) (end 86.75 99.32) (width 0.2) (layer "F.Cu") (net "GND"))
 (segment (start 98.5 99.45) (end 91.06 99.45) (width 0.2) (layer "F.Cu") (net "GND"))
 (segment (start 95.55 93.8) (end 94.05 93.8) (width 0.2) (layer "F.Cu") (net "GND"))
 (segment (start 104.655 90.94) (end 100.364594 90.94) (width 0.2) (layer "F.Cu") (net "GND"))
 (segment (start 91.06 99.45) (end 90.93 99.32) (width 0.2) (layer "F.Cu") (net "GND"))
 (segment (start 88.2 105.6) (end 88.2 100.77) (width 0.2) (layer "F.Cu") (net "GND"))
 (segment (start 90.93 99.32) (end 86.75 99.32) (width 0.2) (layer "F.Cu") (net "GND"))
 (segment (start 105.175 114.3) (end 106 115.125) (width 0.2) (layer "F.Cu") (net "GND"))
 (segment (start 105.34 90.94) (end 104.655 90.94) (width 0.2) (layer "F.Cu") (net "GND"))
 (segment (start 90.93 90.68) (end 86.75 90.68) (width 0.2) (layer "F.Cu") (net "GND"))
 (segment (start 103.2 115.6) (end 103.875 115.6) (width 0.2) (layer "F.Cu") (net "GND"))
 (segment (start 107.825 115.125) (end 108.85 114.1) (width 0.2) (layer "F.Cu") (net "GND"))
 (segment (start 98.1 99.85) (end 98.5 99.45) (width 0.2) (layer "F.Cu") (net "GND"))
 (segment (start 101 105.6) (end 101 104.8) (width 0.2) (layer "F.Cu") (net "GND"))
 (segment (start 122.155 90.94) (end 120.325 90.94) (width 0.2) (layer "F.Cu") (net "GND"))
 (segment (start 106 115.125) (end 107.825 115.125) (width 0.2) (layer "F.Cu") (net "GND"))
 (segment (start 111.52 98.16) (end 111.52 99.58) (width 0.2) (layer "F.Cu") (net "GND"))
 (segment (start 94.05 93.8) (end 90.93 90.68) (width 0.2) (layer "F.Cu") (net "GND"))
 (segment (start 110.505 96.105) (end 105.34 90.94) (width 0.2) (layer "F.Cu") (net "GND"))
 (segment (start 101 104.8) (end 98.1 101.9) (width 0.2) (layer "F.Cu") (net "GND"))
 (segment (start 120.325 90.94) (end 113.305 97.96) (width 0.2) (layer "F.Cu") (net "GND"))
 (segment (start 103.875 115.6) (end 105.175 114.3) (width 0.2) (layer "F.Cu") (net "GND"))
 (segment (start 98.1 101.9) (end 98.1 99.85) (width 0.2) (layer "F.Cu") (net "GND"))
 (segment (start 110.505 97.96) (end 110.505 96.105) (width 0.2) (layer "F.Cu") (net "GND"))
 (via (at 103.2 115.6) (size 0.6) (drill 0.3) (layers "F.Cu" "B.Cu") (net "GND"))
 (via (at 100.364594 90.94) (size 0.6) (drill 0.3) (layers "F.Cu" "B.Cu") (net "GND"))
 (segment (start 94.125 91.7) (end 94.125 93.6) (width 0.2) (layer "B.Cu") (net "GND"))
 (segment (start 94.075 91.75) (end 94.125 91.7) (width 0.2) (layer "B.Cu") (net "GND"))
 (segment (start 100.364594 94.023054) (end 100.364594 90.94) (width 0.2) (layer "B.Cu") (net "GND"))
 (segment (start 91.845 91.595) (end 90.93 90.68) (width 0.2) (layer "B.Cu") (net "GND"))
 (segment (start 91.845 91.75) (end 94.075 91.75) (width 0.2) (layer "B.Cu") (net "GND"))
 (segment (start 91.845 91.75) (end 91.845 91.595) (width 0.2) (layer "B.Cu") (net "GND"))
 (segment (start 101 105.6) (end 101 113.4) (width 0.2) (layer "B.Cu") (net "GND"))
 (segment (start 91.845 98.405) (end 90.93 99.32) (width 0.2) (layer "B.Cu") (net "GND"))
 (segment (start 101 113.4) (end 103.2 115.6) (width 0.2) (layer "B.Cu") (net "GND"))
 (segment (start 97.55 94) (end 98.325 94.775) (width 0.2) (layer "B.Cu") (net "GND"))
 (segment (start 91.845 98.25) (end 91.845 98.405) (width 0.2) (layer "B.Cu") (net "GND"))
 (segment (start 98.325 94.775) (end 99.612648 94.775) (width 0.2) (layer "B.Cu") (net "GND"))
 (segment (start 94.9 90.925) (end 94.125 91.7) (width 0.2) (layer "B.Cu") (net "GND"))
 (segment (start 100.349594 90.925) (end 94.9 90.925) (width 0.2) (layer "B.Cu") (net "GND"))
 (segment (start 97.575 96.3) (end 97.128718 96.3) (width 0.2) (layer "B.Cu") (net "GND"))
 (segment (start 97.55 94) (end 97.55 94.25) (width 0.2) (layer "B.Cu") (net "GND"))
 (segment (start 97.55 94.25) (end 97.575 94.275) (width 0.2) (layer "B.Cu") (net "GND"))
 (segment (start 86.75 90.68) (end 86.75 99.32) (width 0.2) (layer "B.Cu") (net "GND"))
 (segment (start 97.575 94.275) (end 97.575 96.3) (width 0.2) (layer "B.Cu") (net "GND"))
 (segment (start 100.364594 90.94) (end 100.349594 90.925) (width 0.2) (layer "B.Cu") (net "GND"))
 (segment (start 99.612648 94.775) (end 100.364594 94.023054) (width 0.2) (layer "B.Cu") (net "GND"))
 (segment (start 102.7 111.7) (end 103.65 111.7) (width 0.2) (layer "F.Cu") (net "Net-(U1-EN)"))
 (segment (start 103.2 94.405) (end 103.2 105.836473) (width 0.2) (layer "F.Cu") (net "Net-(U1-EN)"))
 (segment (start 104.655 93.48) (end 104.125 93.48) (width 0.2) (layer "F.Cu") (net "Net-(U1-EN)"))
 (segment (start 103.65 114.275) (end 103.625 114.3) (width 0.2) (layer "F.Cu") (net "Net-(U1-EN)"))
 (segment (start 103.65 111.7) (end 103.65 114.275) (width 0.2) (layer "F.Cu") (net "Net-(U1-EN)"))
 (segment (start 104.125 93.48) (end 103.2 94.405) (width 0.2) (layer "F.Cu") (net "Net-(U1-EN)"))
 (via (at 103.2 105.836473) (size 0.6) (drill 0.3) (layers "F.Cu" "B.Cu") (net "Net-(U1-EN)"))
 (via (at 102.7 111.7) (size 0.6) (drill 0.3) (layers "F.Cu" "B.Cu") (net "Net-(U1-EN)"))
 (segment (start 103.2 105.836473) (end 103.2 111.2) (width 0.2) (layer "B.Cu") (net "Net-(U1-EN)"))
 (segment (start 103.2 111.2) (end 102.7 111.7) (width 0.2) (layer "B.Cu") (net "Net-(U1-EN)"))
 (segment (start 89.9 100.7) (end 89.1 100.7) (width 0.2) (layer "F.Cu") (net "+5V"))
 (segment (start 95.3 98.15) (end 95.55 98.4) (width 0.2) (layer "F.Cu") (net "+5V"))
 (segment (start 95.3 97.35) (end 95.3 98.15) (width 0.2) (layer "F.Cu") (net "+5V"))
 (segment (start 91.1 101.9) (end 89.9 100.7) (width 0.2) (layer "F.Cu") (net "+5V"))
 (via (at 95.3 97.35) (size 0.6) (drill 0.3) (layers "F.Cu" "B.Cu") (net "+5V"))
 (via (at 89.1 100.7) (size 0.6) (drill 0.3) (layers "F.Cu" "B.Cu") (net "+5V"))
 (segment (start 89.1 100.7) (end 89.1 98.235406) (width 0.2) (layer "B.Cu") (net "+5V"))
 (segment (start 91.845 97.45) (end 95.2 97.45) (width 0.2) (layer "B.Cu") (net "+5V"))
 (segment (start 91.845 92.55) (end 91.120001 92.55) (width 0.2) (layer "B.Cu") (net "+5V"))
 (segment (start 95.2 97.45) (end 95.3 97.35) (width 0.2) (layer "B.Cu") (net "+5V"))
 (segment (start 89.1 98.235406) (end 90.017703 97.317703) (width 0.2) (layer "B.Cu") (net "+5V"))
 (segment (start 93.3 92.55) (end 93.3 93.998696) (width 0.2) (layer "B.Cu") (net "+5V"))
 (segment (start 94.9 94.375) (end 95.675 93.6) (width 0.2) (layer "B.Cu") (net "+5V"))
 (segment (start 93.3 93.998696) (end 93.676304 94.375) (width 0.2) (layer "B.Cu") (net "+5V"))
 (segment (start 90.017703 97.317703) (end 90.120406 97.215) (width 0.2) (layer "B.Cu") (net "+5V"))
 (segment (start 90.120406 97.215) (end 91.61 97.215) (width 0.2) (layer "B.Cu") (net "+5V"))
 (segment (start 91.120001 92.55) (end 90.017703 93.652298) (width 0.2) (layer "B.Cu") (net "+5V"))
 (segment (start 91.845 92.55) (end 93.3 92.55) (width 0.2) (layer "B.Cu") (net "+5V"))
 (segment (start 90.017703 93.652298) (end 90.017703 97.317703) (width 0.2) (layer "B.Cu") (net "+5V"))
 (segment (start 93.676304 94.375) (end 94.9 94.375) (width 0.2) (layer "B.Cu") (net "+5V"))
 (segment (start 95.675 93.6) (end 95.675 91.7) (width 0.2) (layer "B.Cu") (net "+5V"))
 (segment (start 91.61 97.215) (end 91.845 97.45) (width 0.2) (layer "B.Cu") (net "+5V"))
 (segment (start 93.6 101.9) (end 93.6 103.399999) (width 0.2) (layer "F.Cu") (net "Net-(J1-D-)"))
 (segment (start 104.655 106.18) (end 103.705 106.18) (width 0.2) (layer "F.Cu") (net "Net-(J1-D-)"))
 (segment (start 103.705 106.18) (end 102.535 107.35) (width 0.2) (layer "F.Cu") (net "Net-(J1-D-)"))
 (segment (start 102.535 107.35) (end 97.550001 107.35) (width 0.2) (layer "F.Cu") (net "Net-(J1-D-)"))
 (segment (start 93.6 103.399999) (end 97.550001 107.35) (width 0.2) (layer "F.Cu") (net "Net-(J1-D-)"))
 (segment (start 95.6 101.9) (end 95.6 101.516116) (width 0.2) (layer "F.Cu") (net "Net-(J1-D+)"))
 (segment (start 103.735 108.37) (end 97.686116 108.37) (width 0.2) (layer "F.Cu") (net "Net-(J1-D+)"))
 (segment (start 93.016116 100.1) (end 92.65 100.466116) (width 0.2) (layer "F.Cu") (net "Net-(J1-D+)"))
 (segment (start 104.655 107.45) (end 103.735 108.37) (width 0.2) (layer "F.Cu") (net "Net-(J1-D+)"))
 (segment (start 92.65 100.466116) (end 92.65 103.333884) (width 0.2) (layer "F.Cu") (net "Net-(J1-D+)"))
 (segment (start 92.65 103.333884) (end 97.686116 108.37) (width 0.2) (layer "F.Cu") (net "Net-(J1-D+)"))
 (segment (start 94.183884 100.1) (end 93.016116 100.1) (width 0.2) (layer "F.Cu") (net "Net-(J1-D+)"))
 (segment (start 95.6 101.516116) (end 94.183884 100.1) (width 0.2) (layer "F.Cu") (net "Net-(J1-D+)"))
 (segment (start 104.02 107.35) (end 104.27 107.1) (width 0.2) (layer "F.Cu") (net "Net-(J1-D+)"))
 (segment (start 93.9 96.6) (end 93.6 96.3) (width 0.2) (layer "F.Cu") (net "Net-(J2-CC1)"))
 (segment (start 93.9 98.6) (end 93.9 96.6) (width 0.2) (layer "F.Cu") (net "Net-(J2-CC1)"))
 (via (at 93.9 98.6) (size 0.6) (drill 0.3) (layers "F.Cu" "B.Cu") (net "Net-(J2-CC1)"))
 (via (at 93.6 96.3) (size 0.6) (drill 0.3) (layers "F.Cu" "B.Cu") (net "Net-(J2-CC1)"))
 (segment (start 93.6 96.3) (end 91.895 96.3) (width 0.2) (layer "B.Cu") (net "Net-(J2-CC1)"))
 (segment (start 91.895 96.3) (end 91.845 96.25) (width 0.2) (layer "B.Cu") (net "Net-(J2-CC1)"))
 (segment (start 99.225 96.3) (end 96.925 98.6) (width 0.2) (layer "B.Cu") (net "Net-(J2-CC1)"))
 (segment (start 96.925 98.6) (end 93.9 98.6) (width 0.2) (layer "B.Cu") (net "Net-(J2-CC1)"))
 (segment (start 91.845 93.25) (end 92.60241 93.25) (width 0.2) (layer "B.Cu") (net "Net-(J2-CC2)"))
 (segment (start 98.425 93.225) (end 99.2 94) (width 0.2) (layer "B.Cu") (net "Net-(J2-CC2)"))
 (segment (start 92.87 94.134382) (end 93.510619 94.775) (width 0.2) (layer "B.Cu") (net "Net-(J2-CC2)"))
 (segment (start 95.680189 94.4) (end 96.8 94.4) (width 0.2) (layer "B.Cu") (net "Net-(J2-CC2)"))
 (segment (start 97.137352 93.225) (end 98.425 93.225) (width 0.2) (layer "B.Cu") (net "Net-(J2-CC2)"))
 (segment (start 96.8 94.4) (end 96.8 93.562352) (width 0.2) (layer "B.Cu") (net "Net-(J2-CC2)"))
 (segment (start 95.305189 94.775) (end 95.680189 94.4) (width 0.2) (layer "B.Cu") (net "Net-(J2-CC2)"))
 (segment (start 92.60241 93.25) (end 92.87 93.51759) (width 0.2) (layer "B.Cu") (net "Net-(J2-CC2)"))
 (segment (start 93.510619 94.775) (end 95.305189 94.775) (width 0.2) (layer "B.Cu") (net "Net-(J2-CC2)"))
 (segment (start 92.87 93.51759) (end 92.87 94.134382) (width 0.2) (layer "B.Cu") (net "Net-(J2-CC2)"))
 (segment (start 96.8 93.562352) (end 97.137352 93.225) (width 0.2) (layer "B.Cu") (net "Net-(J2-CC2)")))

